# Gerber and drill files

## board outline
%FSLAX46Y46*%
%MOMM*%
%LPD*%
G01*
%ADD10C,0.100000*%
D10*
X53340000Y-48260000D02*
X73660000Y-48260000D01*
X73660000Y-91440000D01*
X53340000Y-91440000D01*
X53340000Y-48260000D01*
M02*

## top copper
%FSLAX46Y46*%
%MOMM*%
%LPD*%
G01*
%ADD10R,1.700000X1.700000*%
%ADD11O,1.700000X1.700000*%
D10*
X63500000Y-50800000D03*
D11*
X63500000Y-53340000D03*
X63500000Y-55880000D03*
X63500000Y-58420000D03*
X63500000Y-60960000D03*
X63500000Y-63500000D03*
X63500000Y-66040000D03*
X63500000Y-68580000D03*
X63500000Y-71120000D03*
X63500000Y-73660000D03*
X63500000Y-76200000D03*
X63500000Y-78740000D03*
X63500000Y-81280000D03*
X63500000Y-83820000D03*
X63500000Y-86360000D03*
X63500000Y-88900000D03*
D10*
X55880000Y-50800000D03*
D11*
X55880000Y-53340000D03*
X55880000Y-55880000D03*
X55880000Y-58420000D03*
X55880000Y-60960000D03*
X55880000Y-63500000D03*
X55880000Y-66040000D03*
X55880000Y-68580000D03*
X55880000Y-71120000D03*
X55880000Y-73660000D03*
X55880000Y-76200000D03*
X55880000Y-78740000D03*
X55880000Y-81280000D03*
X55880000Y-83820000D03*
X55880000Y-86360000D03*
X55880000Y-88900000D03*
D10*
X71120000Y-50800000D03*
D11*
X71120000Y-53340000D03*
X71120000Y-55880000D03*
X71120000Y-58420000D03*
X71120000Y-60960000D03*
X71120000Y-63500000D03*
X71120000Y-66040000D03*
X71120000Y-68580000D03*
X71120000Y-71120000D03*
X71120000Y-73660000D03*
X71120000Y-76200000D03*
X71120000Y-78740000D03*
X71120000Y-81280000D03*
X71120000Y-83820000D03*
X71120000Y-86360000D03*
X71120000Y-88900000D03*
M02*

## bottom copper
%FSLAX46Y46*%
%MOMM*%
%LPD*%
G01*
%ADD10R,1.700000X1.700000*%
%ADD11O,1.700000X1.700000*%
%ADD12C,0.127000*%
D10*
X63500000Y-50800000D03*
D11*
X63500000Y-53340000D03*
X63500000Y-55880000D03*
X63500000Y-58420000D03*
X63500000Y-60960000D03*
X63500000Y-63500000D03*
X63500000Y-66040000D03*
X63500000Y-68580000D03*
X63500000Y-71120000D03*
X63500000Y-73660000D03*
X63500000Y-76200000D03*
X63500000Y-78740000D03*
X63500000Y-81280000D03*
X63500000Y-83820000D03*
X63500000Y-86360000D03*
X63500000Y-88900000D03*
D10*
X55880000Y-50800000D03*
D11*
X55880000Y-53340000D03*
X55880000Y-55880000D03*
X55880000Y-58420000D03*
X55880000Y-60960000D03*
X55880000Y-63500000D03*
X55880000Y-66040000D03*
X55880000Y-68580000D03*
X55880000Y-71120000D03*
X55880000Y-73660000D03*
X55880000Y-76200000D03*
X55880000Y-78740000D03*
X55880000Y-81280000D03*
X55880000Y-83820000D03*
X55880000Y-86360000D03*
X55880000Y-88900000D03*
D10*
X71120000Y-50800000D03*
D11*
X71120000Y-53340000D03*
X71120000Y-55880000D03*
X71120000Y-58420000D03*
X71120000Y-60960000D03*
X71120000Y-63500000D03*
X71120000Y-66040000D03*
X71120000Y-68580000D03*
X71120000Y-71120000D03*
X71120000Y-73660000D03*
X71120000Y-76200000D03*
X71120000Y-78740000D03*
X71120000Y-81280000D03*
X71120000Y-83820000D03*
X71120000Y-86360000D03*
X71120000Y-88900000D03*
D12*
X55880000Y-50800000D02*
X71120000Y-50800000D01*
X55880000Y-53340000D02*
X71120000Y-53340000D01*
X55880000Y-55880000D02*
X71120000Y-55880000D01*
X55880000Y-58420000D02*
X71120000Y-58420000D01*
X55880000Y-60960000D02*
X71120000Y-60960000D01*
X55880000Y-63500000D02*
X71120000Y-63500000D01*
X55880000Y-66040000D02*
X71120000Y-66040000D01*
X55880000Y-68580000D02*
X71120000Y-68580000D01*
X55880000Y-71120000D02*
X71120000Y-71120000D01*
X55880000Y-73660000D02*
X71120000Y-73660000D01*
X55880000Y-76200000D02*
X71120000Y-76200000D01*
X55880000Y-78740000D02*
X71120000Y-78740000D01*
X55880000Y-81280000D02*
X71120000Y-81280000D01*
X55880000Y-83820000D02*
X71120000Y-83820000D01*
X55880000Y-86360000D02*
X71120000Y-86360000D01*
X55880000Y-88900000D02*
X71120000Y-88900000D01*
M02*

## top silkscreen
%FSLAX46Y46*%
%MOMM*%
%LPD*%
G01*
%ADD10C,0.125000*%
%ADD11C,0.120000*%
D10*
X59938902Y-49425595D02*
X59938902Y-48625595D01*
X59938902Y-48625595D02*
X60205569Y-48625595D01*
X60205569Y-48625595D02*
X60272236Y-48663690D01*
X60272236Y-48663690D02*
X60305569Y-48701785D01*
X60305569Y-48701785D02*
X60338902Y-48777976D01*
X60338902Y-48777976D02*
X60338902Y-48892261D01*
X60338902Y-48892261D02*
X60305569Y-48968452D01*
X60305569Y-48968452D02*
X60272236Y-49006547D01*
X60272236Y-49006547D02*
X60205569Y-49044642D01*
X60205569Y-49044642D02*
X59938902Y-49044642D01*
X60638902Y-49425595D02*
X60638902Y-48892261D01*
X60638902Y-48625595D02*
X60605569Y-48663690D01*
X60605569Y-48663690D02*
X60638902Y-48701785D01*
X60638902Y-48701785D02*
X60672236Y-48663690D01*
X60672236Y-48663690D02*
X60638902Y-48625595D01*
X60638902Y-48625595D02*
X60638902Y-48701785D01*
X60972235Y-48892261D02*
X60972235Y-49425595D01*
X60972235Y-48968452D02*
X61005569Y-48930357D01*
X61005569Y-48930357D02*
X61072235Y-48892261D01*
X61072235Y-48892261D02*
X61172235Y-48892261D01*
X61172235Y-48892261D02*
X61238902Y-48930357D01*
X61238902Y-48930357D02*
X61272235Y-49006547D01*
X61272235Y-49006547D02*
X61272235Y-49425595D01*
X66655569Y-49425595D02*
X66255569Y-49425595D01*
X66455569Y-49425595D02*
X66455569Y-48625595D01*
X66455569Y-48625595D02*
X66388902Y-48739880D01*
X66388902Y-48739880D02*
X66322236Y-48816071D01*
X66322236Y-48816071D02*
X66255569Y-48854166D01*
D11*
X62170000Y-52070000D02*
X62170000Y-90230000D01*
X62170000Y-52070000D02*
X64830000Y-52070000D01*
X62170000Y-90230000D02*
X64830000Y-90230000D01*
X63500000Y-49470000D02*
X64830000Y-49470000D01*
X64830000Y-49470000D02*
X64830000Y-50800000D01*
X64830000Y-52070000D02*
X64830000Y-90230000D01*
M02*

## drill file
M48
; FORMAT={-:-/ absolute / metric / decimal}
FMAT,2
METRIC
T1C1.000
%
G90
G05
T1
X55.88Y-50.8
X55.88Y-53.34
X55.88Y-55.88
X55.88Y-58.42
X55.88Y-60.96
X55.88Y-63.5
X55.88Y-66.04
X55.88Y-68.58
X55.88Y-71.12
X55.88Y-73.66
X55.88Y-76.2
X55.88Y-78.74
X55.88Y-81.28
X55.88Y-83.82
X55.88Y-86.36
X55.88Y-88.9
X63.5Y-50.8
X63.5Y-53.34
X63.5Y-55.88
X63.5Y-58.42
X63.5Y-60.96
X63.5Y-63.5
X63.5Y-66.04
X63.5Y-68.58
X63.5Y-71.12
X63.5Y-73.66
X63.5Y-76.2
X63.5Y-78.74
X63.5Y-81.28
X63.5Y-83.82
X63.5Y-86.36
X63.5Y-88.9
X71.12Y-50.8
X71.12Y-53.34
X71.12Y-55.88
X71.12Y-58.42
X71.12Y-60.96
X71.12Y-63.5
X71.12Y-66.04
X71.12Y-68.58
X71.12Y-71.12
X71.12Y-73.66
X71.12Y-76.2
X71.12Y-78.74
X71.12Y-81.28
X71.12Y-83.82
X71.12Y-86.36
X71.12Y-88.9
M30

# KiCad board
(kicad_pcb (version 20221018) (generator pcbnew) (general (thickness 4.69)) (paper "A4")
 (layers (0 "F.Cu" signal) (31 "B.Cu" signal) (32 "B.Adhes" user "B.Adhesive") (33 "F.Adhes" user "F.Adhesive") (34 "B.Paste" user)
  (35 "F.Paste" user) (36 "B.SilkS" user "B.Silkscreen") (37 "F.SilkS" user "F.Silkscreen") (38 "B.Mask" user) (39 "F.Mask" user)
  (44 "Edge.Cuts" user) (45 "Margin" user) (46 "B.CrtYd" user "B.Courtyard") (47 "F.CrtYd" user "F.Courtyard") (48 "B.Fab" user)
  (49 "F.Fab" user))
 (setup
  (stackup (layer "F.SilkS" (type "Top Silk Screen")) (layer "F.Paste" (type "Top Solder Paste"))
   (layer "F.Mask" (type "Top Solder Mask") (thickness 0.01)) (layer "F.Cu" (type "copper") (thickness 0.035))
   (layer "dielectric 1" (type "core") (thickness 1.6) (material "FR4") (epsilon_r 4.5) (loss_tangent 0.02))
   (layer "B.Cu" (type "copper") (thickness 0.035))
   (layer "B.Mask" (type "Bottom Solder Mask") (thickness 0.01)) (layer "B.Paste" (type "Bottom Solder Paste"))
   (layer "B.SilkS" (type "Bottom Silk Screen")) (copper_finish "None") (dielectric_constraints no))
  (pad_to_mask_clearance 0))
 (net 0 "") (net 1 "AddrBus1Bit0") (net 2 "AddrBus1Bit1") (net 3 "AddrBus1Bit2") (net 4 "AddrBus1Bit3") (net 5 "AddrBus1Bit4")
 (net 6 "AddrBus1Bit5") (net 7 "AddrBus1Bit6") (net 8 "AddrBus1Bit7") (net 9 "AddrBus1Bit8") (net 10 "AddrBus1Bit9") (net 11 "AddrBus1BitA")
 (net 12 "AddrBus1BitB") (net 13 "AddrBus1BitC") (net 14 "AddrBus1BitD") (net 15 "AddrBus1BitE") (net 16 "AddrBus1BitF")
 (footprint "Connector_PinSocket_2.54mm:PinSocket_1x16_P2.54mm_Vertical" (layer "F.Cu") (at 63.5 50.8)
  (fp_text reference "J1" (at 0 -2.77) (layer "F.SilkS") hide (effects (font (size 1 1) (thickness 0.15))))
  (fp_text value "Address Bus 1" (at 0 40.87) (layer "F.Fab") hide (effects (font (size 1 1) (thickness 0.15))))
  (fp_line (start -1.33 1.27) (end -1.33 39.43) (stroke (width 0.12) (type solid)) (layer "F.SilkS"))
  (fp_line (start -1.33 1.27) (end 1.33 1.27) (stroke (width 0.12) (type solid)) (layer "F.SilkS"))
  (fp_line (start -1.33 39.43) (end 1.33 39.43) (stroke (width 0.12) (type solid)) (layer "F.SilkS"))
  (fp_line (start 0 -1.33) (end 1.33 -1.33) (stroke (width 0.12) (type solid)) (layer "F.SilkS"))
  (fp_line (start 1.33 -1.33) (end 1.33 0) (stroke (width 0.12) (type solid)) (layer "F.SilkS"))
  (fp_line (start 1.33 1.27) (end 1.33 39.43) (stroke (width 0.12) (type solid)) (layer "F.SilkS"))
  (pad "1" thru_hole rect (at 0 0) (size 1.7 1.7) (drill 1) (layers "*.Cu" "*.Mask") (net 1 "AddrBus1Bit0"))
  (pad "2" thru_hole oval (at 0 2.54) (size 1.7 1.7) (drill 1) (layers "*.Cu" "*.Mask") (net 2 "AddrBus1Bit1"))
  (pad "3" thru_hole oval (at 0 5.08) (size 1.7 1.7) (drill 1) (layers "*.Cu" "*.Mask") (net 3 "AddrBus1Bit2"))
  (pad "4" thru_hole oval (at 0 7.62) (size 1.7 1.7) (drill 1) (layers "*.Cu" "*.Mask") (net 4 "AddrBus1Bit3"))
  (pad "5" thru_hole oval (at 0 10.16) (size 1.7 1.7) (drill 1) (layers "*.Cu" "*.Mask") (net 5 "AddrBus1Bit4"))
  (pad "6" thru_hole oval (at 0 12.7) (size 1.7 1.7) (drill 1) (layers "*.Cu" "*.Mask") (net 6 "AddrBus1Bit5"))
  (pad "7" thru_hole oval (at 0 15.24) (size 1.7 1.7) (drill 1) (layers "*.Cu" "*.Mask") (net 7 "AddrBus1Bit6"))
  (pad "8" thru_hole oval (at 0 17.78) (size 1.7 1.7) (drill 1) (layers "*.Cu" "*.Mask") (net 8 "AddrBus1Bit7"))
  (pad "9" thru_hole oval (at 0 20.32) (size 1.7 1.7) (drill 1) (layers "*.Cu" "*.Mask") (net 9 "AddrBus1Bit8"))
  (pad "10" thru_hole oval (at 0 22.86) (size 1.7 1.7) (drill 1) (layers "*.Cu" "*.Mask") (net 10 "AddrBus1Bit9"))
  (pad "11" thru_hole oval (at 0 25.4) (size 1.7 1.7) (drill 1) (layers "*.Cu" "*.Mask") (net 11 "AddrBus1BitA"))
  (pad "12" thru_hole oval (at 0 27.94) (size 1.7 1.7) (drill 1) (layers "*.Cu" "*.Mask") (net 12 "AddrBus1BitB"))
  (pad "13" thru_hole oval (at 0 30.48) (size 1.7 1.7) (drill 1) (layers "*.Cu" "*.Mask") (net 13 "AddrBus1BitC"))
  (pad "14" thru_hole oval (at 0 33.02) (size 1.7 1.7) (drill 1) (layers "*.Cu" "*.Mask") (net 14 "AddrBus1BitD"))
  (pad "15" thru_hole oval (at 0 35.56) (size 1.7 1.7) (drill 1) (layers "*.Cu" "*.Mask") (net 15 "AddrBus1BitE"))
  (pad "16" thru_hole oval (at 0 38.1) (size 1.7 1.7) (drill 1) (layers "*.Cu" "*.Mask") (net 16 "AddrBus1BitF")))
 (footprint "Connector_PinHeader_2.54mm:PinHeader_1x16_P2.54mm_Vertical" (layer "B.Cu") (at 55.88 50.8 180)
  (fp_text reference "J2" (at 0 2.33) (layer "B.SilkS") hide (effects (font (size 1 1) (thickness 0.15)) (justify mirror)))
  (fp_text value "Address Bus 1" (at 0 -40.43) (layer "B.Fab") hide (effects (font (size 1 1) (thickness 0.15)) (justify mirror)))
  (pad "1" thru_hole rect (at 0 0 180) (size 1.7 1.7) (drill 1) (layers "*.Cu" "*.Mask") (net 1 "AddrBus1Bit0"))
  (pad "2" thru_hole oval (at 0 -2.54 180) (size 1.7 1.7) (drill 1) (layers "*.Cu" "*.Mask") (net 2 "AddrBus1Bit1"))
  (pad "3" thru_hole oval (at 0 -5.08 180) (size 1.7 1.7) (drill 1) (layers "*.Cu" "*.Mask") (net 3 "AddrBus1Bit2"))
  (pad "4" thru_hole oval (at 0 -7.62 180) (size 1.7 1.7) (drill 1) (layers "*.Cu" "*.Mask") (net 4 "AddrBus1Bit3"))
  (pad "5" thru_hole oval (at 0 -10.16 180) (size 1.7 1.7) (drill 1) (layers "*.Cu" "*.Mask") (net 5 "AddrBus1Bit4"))
  (pad "6" thru_hole oval (at 0 -12.7 180) (size 1.7 1.7) (drill 1) (layers "*.Cu" "*.Mask") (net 6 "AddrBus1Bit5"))
  (pad "7" thru_hole oval (at 0 -15.24 180) (size 1.7 1.7) (drill 1) (layers "*.Cu" "*.Mask") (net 7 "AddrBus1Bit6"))
  (pad "8" thru_hole oval (at 0 -17.78 180) (size 1.7 1.7) (drill 1) (layers "*.Cu" "*.Mask") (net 8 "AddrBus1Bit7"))
  (pad "9" thru_hole oval (at 0 -20.32 180) (size 1.7 1.7) (drill 1) (layers "*.Cu" "*.Mask") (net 9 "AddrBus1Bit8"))
  (pad "10" thru_hole oval (at 0 -22.86 180) (size 1.7 1.7) (drill 1) (layers "*.Cu" "*.Mask") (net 10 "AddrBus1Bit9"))
  (pad "11" thru_hole oval (at 0 -25.4 180) (size 1.7 1.7) (drill 1) (layers "*.Cu" "*.Mask") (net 11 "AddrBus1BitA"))
  (pad "12" thru_hole oval (at 0 -27.94 180) (size 1.7 1.7) (drill 1) (layers "*.Cu" "*.Mask") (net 12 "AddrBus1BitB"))
  (pad "13" thru_hole oval (at 0 -30.48 180) (size 1.7 1.7) (drill 1) (layers "*.Cu" "*.Mask") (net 13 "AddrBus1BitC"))
  (pad "14" thru_hole oval (at 0 -33.02 180) (size 1.7 1.7) (drill 1) (layers "*.Cu" "*.Mask") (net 14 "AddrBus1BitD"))
  (pad "15" thru_hole oval (at 0 -35.56 180) (size 1.7 1.7) (drill 1) (layers "*.Cu" "*.Mask") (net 15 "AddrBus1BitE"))
  (pad "16" thru_hole oval (at 0 -38.1 180) (size 1.7 1.7) (drill 1) (layers "*.Cu" "*.Mask") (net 16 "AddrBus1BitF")))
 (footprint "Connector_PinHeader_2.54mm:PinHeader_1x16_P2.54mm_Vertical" (layer "B.Cu") (at 71.12 50.8 180)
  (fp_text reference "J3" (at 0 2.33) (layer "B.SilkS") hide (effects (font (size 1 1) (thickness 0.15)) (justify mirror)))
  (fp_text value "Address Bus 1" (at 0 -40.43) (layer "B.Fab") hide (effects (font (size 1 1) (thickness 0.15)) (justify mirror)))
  (pad "1" thru_hole rect (at 0 0 180) (size 1.7 1.7) (drill 1) (layers "*.Cu" "*.Mask") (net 1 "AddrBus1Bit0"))
  (pad "2" thru_hole oval (at 0 -2.54 180) (size 1.7 1.7) (drill 1) (layers "*.Cu" "*.Mask") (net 2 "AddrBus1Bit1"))
  (pad "3" thru_hole oval (at 0 -5.08 180) (size 1.7 1.7) (drill 1) (layers "*.Cu" "*.Mask") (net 3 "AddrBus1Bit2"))
  (pad "4" thru_hole oval (at 0 -7.62 180) (size 1.7 1.7) (drill 1) (layers "*.Cu" "*.Mask") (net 4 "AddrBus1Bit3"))
  (pad "5" thru_hole oval (at 0 -10.16 180) (size 1.7 1.7) (drill 1) (layers "*.Cu" "*.Mask") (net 5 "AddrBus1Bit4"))
  (pad "6" thru_hole oval (at 0 -12.7 180) (size 1.7 1.7) (drill 1) (layers "*.Cu" "*.Mask") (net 6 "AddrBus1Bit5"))
  (pad "7" thru_hole oval (at 0 -15.24 180) (size 1.7 1.7) (drill 1) (layers "*.Cu" "*.Mask") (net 7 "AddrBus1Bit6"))
  (pad "8" thru_hole oval (at 0 -17.78 180) (size 1.7 1.7) (drill 1) (layers "*.Cu" "*.Mask") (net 8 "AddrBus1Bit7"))
  (pad "9" thru_hole oval (at 0 -20.32 180) (size 1.7 1.7) (drill 1) (layers "*.Cu" "*.Mask") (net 9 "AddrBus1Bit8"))
  (pad "10" thru_hole oval (at 0 -22.86 180) (size 1.7 1.7) (drill 1) (layers "*.Cu" "*.Mask") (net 10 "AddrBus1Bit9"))
  (pad "11" thru_hole oval (at 0 -25.4 180) (size 1.7 1.7) (drill 1) (layers "*.Cu" "*.Mask") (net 11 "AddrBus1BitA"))
  (pad "12" thru_hole oval (at 0 -27.94 180) (size 1.7 1.7) (drill 1) (layers "*.Cu" "*.Mask") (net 12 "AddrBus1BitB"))
  (pad "13" thru_hole oval (at 0 -30.48 180) (size 1.7 1.7) (drill 1) (layers "*.Cu" "*.Mask") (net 13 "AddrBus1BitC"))
  (pad "14" thru_hole oval (at 0 -33.02 180) (size 1.7 1.7) (drill 1) (layers "*.Cu" "*.Mask") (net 14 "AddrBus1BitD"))
  (pad "15" thru_hole oval (at 0 -35.56 180) (size 1.7 1.7) (drill 1) (layers "*.Cu" "*.Mask") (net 15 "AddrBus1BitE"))
  (pad "16" thru_hole oval (at 0 -38.1 180) (size 1.7 1.7) (drill 1) (layers "*.Cu" "*.Mask") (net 16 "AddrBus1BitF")))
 (gr_rect (start 53.34 48.26) (end 73.66 91.44) (stroke (width 0.1) (type default)) (fill none) (layer "Edge.Cuts"))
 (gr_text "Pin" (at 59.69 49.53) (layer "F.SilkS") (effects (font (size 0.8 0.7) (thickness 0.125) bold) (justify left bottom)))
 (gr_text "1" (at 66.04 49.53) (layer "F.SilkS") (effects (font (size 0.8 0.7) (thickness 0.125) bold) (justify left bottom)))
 (segment (start 55.88 50.8) (end 71.12 50.8) (width 0.127) (layer "B.Cu") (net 1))
 (segment (start 55.88 53.34) (end 71.12 53.34) (width 0.127) (layer "B.Cu") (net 2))
 (segment (start 55.88 55.88) (end 71.12 55.88) (width 0.127) (layer "B.Cu") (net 3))
 (segment (start 55.88 58.42) (end 71.12 58.42) (width 0.127) (layer "B.Cu") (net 4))
 (segment (start 55.88 60.96) (end 71.12 60.96) (width 0.127) (layer "B.Cu") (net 5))
 (segment (start 55.88 63.5) (end 71.12 63.5) (width 0.127) (layer "B.Cu") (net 6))
 (segment (start 55.88 66.04) (end 71.12 66.04) (width 0.127) (layer "B.Cu") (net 7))
 (segment (start 55.88 68.58) (end 71.12 68.58) (width 0.127) (layer "B.Cu") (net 8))
 (segment (start 55.88 71.12) (end 71.12 71.12) (width 0.127) (layer "B.Cu") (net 9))
 (segment (start 55.88 73.66) (end 71.12 73.66) (width 0.127) (layer "B.Cu") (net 10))
 (segment (start 55.88 76.2) (end 71.12 76.2) (width 0.127) (layer "B.Cu") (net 11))
 (segment (start 55.88 78.74) (end 71.12 78.74) (width 0.127) (layer "B.Cu") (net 12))
 (segment (start 55.88 81.28) (end 71.12 81.28) (width 0.127) (layer "B.Cu") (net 13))
 (segment (start 55.88 83.82) (end 71.12 83.82) (width 0.127) (layer "B.Cu") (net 14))
 (segment (start 55.88 86.36) (end 71.12 86.36) (width 0.127) (layer "B.Cu") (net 15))
 (segment (start 55.88 88.9) (end 71.12 88.9) (width 0.127) (layer "B.Cu") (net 16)))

